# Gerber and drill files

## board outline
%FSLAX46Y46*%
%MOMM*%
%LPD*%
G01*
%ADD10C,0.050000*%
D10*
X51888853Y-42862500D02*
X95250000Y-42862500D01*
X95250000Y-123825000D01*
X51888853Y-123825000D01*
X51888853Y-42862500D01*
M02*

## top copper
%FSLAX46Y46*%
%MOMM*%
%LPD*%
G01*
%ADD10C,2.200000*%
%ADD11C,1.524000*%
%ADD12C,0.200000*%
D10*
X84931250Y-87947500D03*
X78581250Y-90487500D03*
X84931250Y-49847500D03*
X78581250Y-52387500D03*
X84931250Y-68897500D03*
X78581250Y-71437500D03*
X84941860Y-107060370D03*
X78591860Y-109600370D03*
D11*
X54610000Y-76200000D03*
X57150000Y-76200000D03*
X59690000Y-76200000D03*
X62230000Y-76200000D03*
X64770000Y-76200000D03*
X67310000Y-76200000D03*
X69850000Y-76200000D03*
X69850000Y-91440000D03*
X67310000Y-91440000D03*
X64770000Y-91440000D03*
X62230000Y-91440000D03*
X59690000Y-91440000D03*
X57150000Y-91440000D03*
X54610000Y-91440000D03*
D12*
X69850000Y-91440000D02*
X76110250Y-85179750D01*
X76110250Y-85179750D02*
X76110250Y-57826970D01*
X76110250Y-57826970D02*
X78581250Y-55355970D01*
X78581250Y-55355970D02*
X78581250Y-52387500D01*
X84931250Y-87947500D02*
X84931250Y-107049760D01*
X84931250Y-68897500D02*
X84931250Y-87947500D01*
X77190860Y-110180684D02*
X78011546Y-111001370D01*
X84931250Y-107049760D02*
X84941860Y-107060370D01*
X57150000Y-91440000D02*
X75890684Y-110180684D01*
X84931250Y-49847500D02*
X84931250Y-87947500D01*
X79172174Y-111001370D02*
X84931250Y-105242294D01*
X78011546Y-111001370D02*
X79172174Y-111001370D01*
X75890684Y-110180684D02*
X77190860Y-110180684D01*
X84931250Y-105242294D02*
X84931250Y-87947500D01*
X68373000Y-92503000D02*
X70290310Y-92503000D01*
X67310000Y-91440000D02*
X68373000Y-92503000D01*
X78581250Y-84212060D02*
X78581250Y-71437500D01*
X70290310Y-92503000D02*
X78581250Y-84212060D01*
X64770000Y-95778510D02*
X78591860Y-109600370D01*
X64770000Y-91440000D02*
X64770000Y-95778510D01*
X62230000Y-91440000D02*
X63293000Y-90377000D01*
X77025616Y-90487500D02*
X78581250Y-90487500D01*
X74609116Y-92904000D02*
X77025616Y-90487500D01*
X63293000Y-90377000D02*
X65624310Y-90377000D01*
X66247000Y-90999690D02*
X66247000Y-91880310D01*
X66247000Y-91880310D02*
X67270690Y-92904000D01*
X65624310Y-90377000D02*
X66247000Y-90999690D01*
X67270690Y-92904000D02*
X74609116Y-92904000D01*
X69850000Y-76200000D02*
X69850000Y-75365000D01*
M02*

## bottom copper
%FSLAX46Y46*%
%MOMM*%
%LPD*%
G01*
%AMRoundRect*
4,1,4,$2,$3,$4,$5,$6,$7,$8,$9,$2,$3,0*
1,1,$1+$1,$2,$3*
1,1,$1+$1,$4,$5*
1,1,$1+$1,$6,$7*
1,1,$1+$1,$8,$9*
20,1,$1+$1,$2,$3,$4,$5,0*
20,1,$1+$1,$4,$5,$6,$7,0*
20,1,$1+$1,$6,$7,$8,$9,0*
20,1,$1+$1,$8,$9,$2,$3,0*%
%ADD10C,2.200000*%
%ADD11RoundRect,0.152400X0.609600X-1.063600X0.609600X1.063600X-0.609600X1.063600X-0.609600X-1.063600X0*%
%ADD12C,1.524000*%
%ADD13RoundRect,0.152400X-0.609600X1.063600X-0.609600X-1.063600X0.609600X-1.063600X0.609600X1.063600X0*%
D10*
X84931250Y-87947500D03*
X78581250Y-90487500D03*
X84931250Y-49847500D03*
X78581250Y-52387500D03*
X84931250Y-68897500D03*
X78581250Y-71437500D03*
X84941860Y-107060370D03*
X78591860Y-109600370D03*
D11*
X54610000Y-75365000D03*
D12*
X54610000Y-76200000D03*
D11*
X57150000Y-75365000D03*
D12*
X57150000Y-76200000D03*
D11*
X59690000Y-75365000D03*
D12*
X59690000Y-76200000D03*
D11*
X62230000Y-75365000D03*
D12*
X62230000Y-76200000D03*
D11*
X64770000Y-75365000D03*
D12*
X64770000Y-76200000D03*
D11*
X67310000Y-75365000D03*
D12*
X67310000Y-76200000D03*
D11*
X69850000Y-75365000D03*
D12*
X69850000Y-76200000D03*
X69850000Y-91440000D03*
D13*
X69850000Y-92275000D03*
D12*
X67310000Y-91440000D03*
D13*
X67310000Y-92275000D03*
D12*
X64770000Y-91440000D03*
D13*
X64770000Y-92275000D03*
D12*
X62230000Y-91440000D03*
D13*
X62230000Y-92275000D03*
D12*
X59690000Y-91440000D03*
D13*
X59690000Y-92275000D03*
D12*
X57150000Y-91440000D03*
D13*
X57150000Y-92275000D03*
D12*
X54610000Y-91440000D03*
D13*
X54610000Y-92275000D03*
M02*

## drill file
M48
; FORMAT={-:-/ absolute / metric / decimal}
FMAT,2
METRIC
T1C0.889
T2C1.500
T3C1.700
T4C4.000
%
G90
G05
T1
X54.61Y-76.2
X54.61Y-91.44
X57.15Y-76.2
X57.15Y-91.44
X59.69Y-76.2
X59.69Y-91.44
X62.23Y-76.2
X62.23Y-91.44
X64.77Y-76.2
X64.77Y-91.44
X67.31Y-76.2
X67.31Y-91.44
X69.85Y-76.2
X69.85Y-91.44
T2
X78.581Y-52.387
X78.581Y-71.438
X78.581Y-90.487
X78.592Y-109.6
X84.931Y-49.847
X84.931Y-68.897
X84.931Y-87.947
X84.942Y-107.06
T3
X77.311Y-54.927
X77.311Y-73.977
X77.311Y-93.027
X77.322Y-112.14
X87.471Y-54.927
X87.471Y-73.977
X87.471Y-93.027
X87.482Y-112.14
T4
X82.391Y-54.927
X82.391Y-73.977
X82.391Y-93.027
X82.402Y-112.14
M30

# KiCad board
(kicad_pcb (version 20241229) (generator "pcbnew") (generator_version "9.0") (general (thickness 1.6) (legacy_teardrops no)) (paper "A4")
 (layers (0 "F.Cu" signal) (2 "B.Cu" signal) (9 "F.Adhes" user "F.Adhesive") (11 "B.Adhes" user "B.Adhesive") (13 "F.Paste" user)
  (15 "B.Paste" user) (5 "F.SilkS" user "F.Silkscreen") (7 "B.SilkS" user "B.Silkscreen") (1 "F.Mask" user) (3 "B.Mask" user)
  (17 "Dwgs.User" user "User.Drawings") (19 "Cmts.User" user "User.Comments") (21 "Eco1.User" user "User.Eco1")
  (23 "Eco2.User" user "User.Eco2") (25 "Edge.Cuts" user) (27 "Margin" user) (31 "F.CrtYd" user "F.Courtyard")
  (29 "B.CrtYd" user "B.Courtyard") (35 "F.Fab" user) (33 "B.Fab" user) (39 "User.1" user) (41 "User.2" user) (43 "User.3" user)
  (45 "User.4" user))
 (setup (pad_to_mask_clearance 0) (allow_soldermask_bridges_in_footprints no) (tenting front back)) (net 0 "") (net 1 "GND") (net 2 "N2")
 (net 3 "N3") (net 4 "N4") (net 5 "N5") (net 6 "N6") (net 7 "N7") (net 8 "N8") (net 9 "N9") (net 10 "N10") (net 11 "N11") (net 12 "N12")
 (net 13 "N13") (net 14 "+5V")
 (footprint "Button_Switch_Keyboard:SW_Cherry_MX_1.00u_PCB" (layer "F.Cu") (at 84.93125 87.9475)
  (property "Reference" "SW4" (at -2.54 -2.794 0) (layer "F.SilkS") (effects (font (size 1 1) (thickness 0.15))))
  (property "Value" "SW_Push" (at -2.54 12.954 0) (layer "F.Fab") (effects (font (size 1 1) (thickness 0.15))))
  (pad "" np_thru_hole circle (at -7.62 5.08) (size 1.7 1.7) (drill 1.7) (layers "*.Cu" "*.Mask"))
  (pad "" np_thru_hole circle (at -2.54 5.08) (size 4 4) (drill 4) (layers "*.Cu" "*.Mask"))
  (pad "" np_thru_hole circle (at 2.54 5.08) (size 1.7 1.7) (drill 1.7) (layers "*.Cu" "*.Mask"))
  (pad "1" thru_hole circle (at 0 0) (size 2.2 2.2) (drill 1.5) (layers "*.Cu" "*.Mask") (remove_unused_layers no) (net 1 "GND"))
  (pad "2" thru_hole circle (at -6.35 2.54) (size 2.2 2.2) (drill 1.5) (layers "*.Cu" "*.Mask") (remove_unused_layers no) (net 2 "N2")))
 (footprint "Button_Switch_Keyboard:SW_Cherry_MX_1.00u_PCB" (layer "F.Cu") (at 84.93125 49.8475)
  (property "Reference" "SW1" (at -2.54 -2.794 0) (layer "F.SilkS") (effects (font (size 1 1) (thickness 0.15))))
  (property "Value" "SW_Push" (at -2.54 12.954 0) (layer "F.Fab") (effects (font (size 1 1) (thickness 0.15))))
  (pad "" np_thru_hole circle (at -7.62 5.08) (size 1.7 1.7) (drill 1.7) (layers "*.Cu" "*.Mask"))
  (pad "" np_thru_hole circle (at -2.54 5.08) (size 4 4) (drill 4) (layers "*.Cu" "*.Mask"))
  (pad "" np_thru_hole circle (at 2.54 5.08) (size 1.7 1.7) (drill 1.7) (layers "*.Cu" "*.Mask"))
  (pad "1" thru_hole circle (at 0 0) (size 2.2 2.2) (drill 1.5) (layers "*.Cu" "*.Mask") (remove_unused_layers no) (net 1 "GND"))
  (pad "2" thru_hole circle (at -6.35 2.54) (size 2.2 2.2) (drill 1.5) (layers "*.Cu" "*.Mask") (remove_unused_layers no) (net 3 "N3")))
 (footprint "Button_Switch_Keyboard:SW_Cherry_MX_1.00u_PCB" (layer "F.Cu") (at 84.93125 68.8975)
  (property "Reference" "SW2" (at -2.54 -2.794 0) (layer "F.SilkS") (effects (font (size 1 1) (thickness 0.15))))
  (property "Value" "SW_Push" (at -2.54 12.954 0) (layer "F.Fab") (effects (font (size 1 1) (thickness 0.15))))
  (pad "" np_thru_hole circle (at -7.62 5.08) (size 1.7 1.7) (drill 1.7) (layers "*.Cu" "*.Mask"))
  (pad "" np_thru_hole circle (at -2.54 5.08) (size 4 4) (drill 4) (layers "*.Cu" "*.Mask"))
  (pad "" np_thru_hole circle (at 2.54 5.08) (size 1.7 1.7) (drill 1.7) (layers "*.Cu" "*.Mask"))
  (pad "1" thru_hole circle (at 0 0) (size 2.2 2.2) (drill 1.5) (layers "*.Cu" "*.Mask") (remove_unused_layers no) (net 1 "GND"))
  (pad "2" thru_hole circle (at -6.35 2.54) (size 2.2 2.2) (drill 1.5) (layers "*.Cu" "*.Mask") (remove_unused_layers no) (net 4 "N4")))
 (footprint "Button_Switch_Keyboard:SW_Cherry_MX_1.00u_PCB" (layer "F.Cu") (at 84.94186 107.06037)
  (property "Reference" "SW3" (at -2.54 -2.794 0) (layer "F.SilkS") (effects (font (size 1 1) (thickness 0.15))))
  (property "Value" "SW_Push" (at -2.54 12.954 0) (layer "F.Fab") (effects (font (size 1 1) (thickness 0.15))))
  (pad "" np_thru_hole circle (at -7.62 5.08) (size 1.7 1.7) (drill 1.7) (layers "*.Cu" "*.Mask"))
  (pad "" np_thru_hole circle (at -2.54 5.08) (size 4 4) (drill 4) (layers "*.Cu" "*.Mask"))
  (pad "" np_thru_hole circle (at 2.54 5.08) (size 1.7 1.7) (drill 1.7) (layers "*.Cu" "*.Mask"))
  (pad "1" thru_hole circle (at 0 0) (size 2.2 2.2) (drill 1.5) (layers "*.Cu" "*.Mask") (remove_unused_layers no) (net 1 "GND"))
  (pad "2" thru_hole circle (at -6.35 2.54) (size 2.2 2.2) (drill 1.5) (layers "*.Cu" "*.Mask") (remove_unused_layers no) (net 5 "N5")))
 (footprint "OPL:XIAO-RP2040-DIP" (layer "B.Cu") (at 62.23 83.82 -90)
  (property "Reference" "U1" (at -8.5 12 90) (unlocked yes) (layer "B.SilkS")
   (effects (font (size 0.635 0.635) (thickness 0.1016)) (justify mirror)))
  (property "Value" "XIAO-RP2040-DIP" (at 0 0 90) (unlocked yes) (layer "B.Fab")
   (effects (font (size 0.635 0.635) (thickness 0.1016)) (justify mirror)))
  (pad "1" smd roundrect (at -8.455 7.62 90) (size 2.432 1.524) (layers "B.Cu" "B.Mask") (roundrect_rratio 0.1) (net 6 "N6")
   (thermal_bridge_angle 45))
  (pad "1" thru_hole circle (at -7.62 7.62 90) (size 1.524 1.524) (drill 0.889) (layers "*.Cu" "*.Mask") (remove_unused_layers no)
   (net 6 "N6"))
  (pad "2" smd roundrect (at -8.455 5.08 90) (size 2.432 1.524) (layers "B.Cu" "B.Mask") (roundrect_rratio 0.1) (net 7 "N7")
   (thermal_bridge_angle 45))
  (pad "2" thru_hole circle (at -7.62 5.08 90) (size 1.524 1.524) (drill 0.889) (layers "*.Cu" "*.Mask") (remove_unused_layers no)
   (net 7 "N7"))
  (pad "3" smd roundrect (at -8.455 2.54 90) (size 2.432 1.524) (layers "B.Cu" "B.Mask") (roundrect_rratio 0.1) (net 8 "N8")
   (thermal_bridge_angle 45))
  (pad "3" thru_hole circle (at -7.62 2.54 90) (size 1.524 1.524) (drill 0.889) (layers "*.Cu" "*.Mask") (remove_unused_layers no)
   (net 8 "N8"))
  (pad "4" smd roundrect (at -8.455 0 90) (size 2.432 1.524) (layers "B.Cu" "B.Mask") (roundrect_rratio 0.1) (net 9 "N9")
   (thermal_bridge_angle 45))
  (pad "4" thru_hole circle (at -7.62 0 90) (size 1.524 1.524) (drill 0.889) (layers "*.Cu" "*.Mask") (remove_unused_layers no) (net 9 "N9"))
  (pad "5" smd roundrect (at -8.455 -2.54 90) (size 2.432 1.524) (layers "B.Cu" "B.Mask") (roundrect_rratio 0.1) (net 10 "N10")
   (thermal_bridge_angle 45))
  (pad "5" thru_hole circle (at -7.62 -2.54 90) (size 1.524 1.524) (drill 0.889) (layers "*.Cu" "*.Mask") (remove_unused_layers no)
   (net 10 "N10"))
  (pad "6" smd roundrect (at -8.455 -5.08 90) (size 2.432 1.524) (layers "B.Cu" "B.Mask") (roundrect_rratio 0.1) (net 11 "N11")
   (thermal_bridge_angle 45))
  (pad "6" thru_hole circle (at -7.62 -5.08 90) (size 1.524 1.524) (drill 0.889) (layers "*.Cu" "*.Mask") (remove_unused_layers no)
   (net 11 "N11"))
  (pad "7" smd roundrect (at -8.455 -7.62 90) (size 2.432 1.524) (layers "B.Cu" "B.Mask") (roundrect_rratio 0.1) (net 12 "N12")
   (thermal_bridge_angle 45))
  (pad "7" thru_hole circle (at -7.62 -7.62 90) (size 1.524 1.524) (drill 0.889) (layers "*.Cu" "*.Mask") (remove_unused_layers no)
   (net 12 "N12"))
  (pad "8" thru_hole circle (at 7.62 -7.62 270) (size 1.524 1.524) (drill 0.889) (layers "*.Cu" "*.Mask") (remove_unused_layers no)
   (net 3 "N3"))
  (pad "8" smd roundrect (at 8.455 -7.62 270) (size 2.432 1.524) (layers "B.Cu" "B.Mask") (roundrect_rratio 0.1) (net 3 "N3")
   (thermal_bridge_angle 45))
  (pad "9" thru_hole circle (at 7.62 -5.08 270) (size 1.524 1.524) (drill 0.889) (layers "*.Cu" "*.Mask") (remove_unused_layers no)
   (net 4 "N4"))
  (pad "9" smd roundrect (at 8.455 -5.08 270) (size 2.432 1.524) (layers "B.Cu" "B.Mask") (roundrect_rratio 0.1) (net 4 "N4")
   (thermal_bridge_angle 45))
  (pad "10" thru_hole circle (at 7.62 -2.54 270) (size 1.524 1.524) (drill 0.889) (layers "*.Cu" "*.Mask") (remove_unused_layers no)
   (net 5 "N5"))
  (pad "10" smd roundrect (at 8.455 -2.54 270) (size 2.432 1.524) (layers "B.Cu" "B.Mask") (roundrect_rratio 0.1) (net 5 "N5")
   (thermal_bridge_angle 45))
  (pad "11" thru_hole circle (at 7.62 0 270) (size 1.524 1.524) (drill 0.889) (layers "*.Cu" "*.Mask") (remove_unused_layers no)
   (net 2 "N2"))
  (pad "11" smd roundrect (at 8.455 0 270) (size 2.432 1.524) (layers "B.Cu" "B.Mask") (roundrect_rratio 0.1) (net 2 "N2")
   (thermal_bridge_angle 45))
  (pad "12" thru_hole circle (at 7.62 2.54 270) (size 1.524 1.524) (drill 0.889) (layers "*.Cu" "*.Mask") (remove_unused_layers no)
   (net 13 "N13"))
  (pad "12" smd roundrect (at 8.455 2.54 270) (size 2.432 1.524) (layers "B.Cu" "B.Mask") (roundrect_rratio 0.1) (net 13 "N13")
   (thermal_bridge_angle 45))
  (pad "13" thru_hole circle (at 7.62 5.08 270) (size 1.524 1.524) (drill 0.889) (layers "*.Cu" "*.Mask") (remove_unused_layers no)
   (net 1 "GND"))
  (pad "13" smd roundrect (at 8.455 5.08 270) (size 2.432 1.524) (layers "B.Cu" "B.Mask") (roundrect_rratio 0.1) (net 1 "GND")
   (thermal_bridge_angle 45))
  (pad "14" thru_hole circle (at 7.62 7.62 270) (size 1.524 1.524) (drill 0.889) (layers "*.Cu" "*.Mask") (remove_unused_layers no)
   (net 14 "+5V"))
  (pad "14" smd roundrect (at 8.455 7.62 270) (size 2.432 1.524) (layers "B.Cu" "B.Mask") (roundrect_rratio 0.1) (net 14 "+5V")
   (thermal_bridge_angle 45)))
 (gr_rect (start 51.888853 42.8625) (end 95.25 123.825) (stroke (width 0.05) (type default)) (fill no) (layer "Edge.Cuts"))
 (segment (start 69.85 91.44) (end 76.11025 85.17975) (width 0.2) (layer "F.Cu") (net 3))
 (segment (start 76.11025 85.17975) (end 76.11025 57.82697) (width 0.2) (layer "F.Cu") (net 3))
 (segment (start 76.11025 57.82697) (end 78.58125 55.35597) (width 0.2) (layer "F.Cu") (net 3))
 (segment (start 78.58125 55.35597) (end 78.58125 52.3875) (width 0.2) (layer "F.Cu") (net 3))
 (segment (start 84.93125 87.9475) (end 84.93125 107.04976) (width 0.2) (layer "F.Cu") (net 1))
 (segment (start 84.93125 68.8975) (end 84.93125 87.9475) (width 0.2) (layer "F.Cu") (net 1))
 (segment (start 77.19086 110.180684) (end 78.011546 111.00137) (width 0.2) (layer "F.Cu") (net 1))
 (segment (start 84.93125 107.04976) (end 84.94186 107.06037) (width 0.2) (layer "F.Cu") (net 1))
 (segment (start 57.15 91.44) (end 75.890684 110.180684) (width 0.2) (layer "F.Cu") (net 1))
 (segment (start 84.93125 49.8475) (end 84.93125 87.9475) (width 0.2) (layer "F.Cu") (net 1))
 (segment (start 79.172174 111.00137) (end 84.93125 105.242294) (width 0.2) (layer "F.Cu") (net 1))
 (segment (start 78.011546 111.00137) (end 79.172174 111.00137) (width 0.2) (layer "F.Cu") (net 1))
 (segment (start 75.890684 110.180684) (end 77.19086 110.180684) (width 0.2) (layer "F.Cu") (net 1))
 (segment (start 84.93125 105.242294) (end 84.93125 87.9475) (width 0.2) (layer "F.Cu") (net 1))
 (segment (start 68.373 92.503) (end 70.29031 92.503) (width 0.2) (layer "F.Cu") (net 4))
 (segment (start 67.31 91.44) (end 68.373 92.503) (width 0.2) (layer "F.Cu") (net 4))
 (segment (start 78.58125 84.21206) (end 78.58125 71.4375) (width 0.2) (layer "F.Cu") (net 4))
 (segment (start 70.29031 92.503) (end 78.58125 84.21206) (width 0.2) (layer "F.Cu") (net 4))
 (segment (start 64.77 95.77851) (end 78.59186 109.60037) (width 0.2) (layer "F.Cu") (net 5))
 (segment (start 64.77 91.44) (end 64.77 95.77851) (width 0.2) (layer "F.Cu") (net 5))
 (segment (start 62.23 91.44) (end 63.293 90.377) (width 0.2) (layer "F.Cu") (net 2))
 (segment (start 77.025616 90.4875) (end 78.58125 90.4875) (width 0.2) (layer "F.Cu") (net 2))
 (segment (start 74.609116 92.904) (end 77.025616 90.4875) (width 0.2) (layer "F.Cu") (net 2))
 (segment (start 63.293 90.377) (end 65.62431 90.377) (width 0.2) (layer "F.Cu") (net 2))
 (segment (start 66.247 90.99969) (end 66.247 91.88031) (width 0.2) (layer "F.Cu") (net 2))
 (segment (start 66.247 91.88031) (end 67.27069 92.904) (width 0.2) (layer "F.Cu") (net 2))
 (segment (start 65.62431 90.377) (end 66.247 90.99969) (width 0.2) (layer "F.Cu") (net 2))
 (segment (start 67.27069 92.904) (end 74.609116 92.904) (width 0.2) (layer "F.Cu") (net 2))
 (segment (start 69.85 76.2) (end 69.85 75.365) (width 0.2) (layer "F.Cu") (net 12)))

